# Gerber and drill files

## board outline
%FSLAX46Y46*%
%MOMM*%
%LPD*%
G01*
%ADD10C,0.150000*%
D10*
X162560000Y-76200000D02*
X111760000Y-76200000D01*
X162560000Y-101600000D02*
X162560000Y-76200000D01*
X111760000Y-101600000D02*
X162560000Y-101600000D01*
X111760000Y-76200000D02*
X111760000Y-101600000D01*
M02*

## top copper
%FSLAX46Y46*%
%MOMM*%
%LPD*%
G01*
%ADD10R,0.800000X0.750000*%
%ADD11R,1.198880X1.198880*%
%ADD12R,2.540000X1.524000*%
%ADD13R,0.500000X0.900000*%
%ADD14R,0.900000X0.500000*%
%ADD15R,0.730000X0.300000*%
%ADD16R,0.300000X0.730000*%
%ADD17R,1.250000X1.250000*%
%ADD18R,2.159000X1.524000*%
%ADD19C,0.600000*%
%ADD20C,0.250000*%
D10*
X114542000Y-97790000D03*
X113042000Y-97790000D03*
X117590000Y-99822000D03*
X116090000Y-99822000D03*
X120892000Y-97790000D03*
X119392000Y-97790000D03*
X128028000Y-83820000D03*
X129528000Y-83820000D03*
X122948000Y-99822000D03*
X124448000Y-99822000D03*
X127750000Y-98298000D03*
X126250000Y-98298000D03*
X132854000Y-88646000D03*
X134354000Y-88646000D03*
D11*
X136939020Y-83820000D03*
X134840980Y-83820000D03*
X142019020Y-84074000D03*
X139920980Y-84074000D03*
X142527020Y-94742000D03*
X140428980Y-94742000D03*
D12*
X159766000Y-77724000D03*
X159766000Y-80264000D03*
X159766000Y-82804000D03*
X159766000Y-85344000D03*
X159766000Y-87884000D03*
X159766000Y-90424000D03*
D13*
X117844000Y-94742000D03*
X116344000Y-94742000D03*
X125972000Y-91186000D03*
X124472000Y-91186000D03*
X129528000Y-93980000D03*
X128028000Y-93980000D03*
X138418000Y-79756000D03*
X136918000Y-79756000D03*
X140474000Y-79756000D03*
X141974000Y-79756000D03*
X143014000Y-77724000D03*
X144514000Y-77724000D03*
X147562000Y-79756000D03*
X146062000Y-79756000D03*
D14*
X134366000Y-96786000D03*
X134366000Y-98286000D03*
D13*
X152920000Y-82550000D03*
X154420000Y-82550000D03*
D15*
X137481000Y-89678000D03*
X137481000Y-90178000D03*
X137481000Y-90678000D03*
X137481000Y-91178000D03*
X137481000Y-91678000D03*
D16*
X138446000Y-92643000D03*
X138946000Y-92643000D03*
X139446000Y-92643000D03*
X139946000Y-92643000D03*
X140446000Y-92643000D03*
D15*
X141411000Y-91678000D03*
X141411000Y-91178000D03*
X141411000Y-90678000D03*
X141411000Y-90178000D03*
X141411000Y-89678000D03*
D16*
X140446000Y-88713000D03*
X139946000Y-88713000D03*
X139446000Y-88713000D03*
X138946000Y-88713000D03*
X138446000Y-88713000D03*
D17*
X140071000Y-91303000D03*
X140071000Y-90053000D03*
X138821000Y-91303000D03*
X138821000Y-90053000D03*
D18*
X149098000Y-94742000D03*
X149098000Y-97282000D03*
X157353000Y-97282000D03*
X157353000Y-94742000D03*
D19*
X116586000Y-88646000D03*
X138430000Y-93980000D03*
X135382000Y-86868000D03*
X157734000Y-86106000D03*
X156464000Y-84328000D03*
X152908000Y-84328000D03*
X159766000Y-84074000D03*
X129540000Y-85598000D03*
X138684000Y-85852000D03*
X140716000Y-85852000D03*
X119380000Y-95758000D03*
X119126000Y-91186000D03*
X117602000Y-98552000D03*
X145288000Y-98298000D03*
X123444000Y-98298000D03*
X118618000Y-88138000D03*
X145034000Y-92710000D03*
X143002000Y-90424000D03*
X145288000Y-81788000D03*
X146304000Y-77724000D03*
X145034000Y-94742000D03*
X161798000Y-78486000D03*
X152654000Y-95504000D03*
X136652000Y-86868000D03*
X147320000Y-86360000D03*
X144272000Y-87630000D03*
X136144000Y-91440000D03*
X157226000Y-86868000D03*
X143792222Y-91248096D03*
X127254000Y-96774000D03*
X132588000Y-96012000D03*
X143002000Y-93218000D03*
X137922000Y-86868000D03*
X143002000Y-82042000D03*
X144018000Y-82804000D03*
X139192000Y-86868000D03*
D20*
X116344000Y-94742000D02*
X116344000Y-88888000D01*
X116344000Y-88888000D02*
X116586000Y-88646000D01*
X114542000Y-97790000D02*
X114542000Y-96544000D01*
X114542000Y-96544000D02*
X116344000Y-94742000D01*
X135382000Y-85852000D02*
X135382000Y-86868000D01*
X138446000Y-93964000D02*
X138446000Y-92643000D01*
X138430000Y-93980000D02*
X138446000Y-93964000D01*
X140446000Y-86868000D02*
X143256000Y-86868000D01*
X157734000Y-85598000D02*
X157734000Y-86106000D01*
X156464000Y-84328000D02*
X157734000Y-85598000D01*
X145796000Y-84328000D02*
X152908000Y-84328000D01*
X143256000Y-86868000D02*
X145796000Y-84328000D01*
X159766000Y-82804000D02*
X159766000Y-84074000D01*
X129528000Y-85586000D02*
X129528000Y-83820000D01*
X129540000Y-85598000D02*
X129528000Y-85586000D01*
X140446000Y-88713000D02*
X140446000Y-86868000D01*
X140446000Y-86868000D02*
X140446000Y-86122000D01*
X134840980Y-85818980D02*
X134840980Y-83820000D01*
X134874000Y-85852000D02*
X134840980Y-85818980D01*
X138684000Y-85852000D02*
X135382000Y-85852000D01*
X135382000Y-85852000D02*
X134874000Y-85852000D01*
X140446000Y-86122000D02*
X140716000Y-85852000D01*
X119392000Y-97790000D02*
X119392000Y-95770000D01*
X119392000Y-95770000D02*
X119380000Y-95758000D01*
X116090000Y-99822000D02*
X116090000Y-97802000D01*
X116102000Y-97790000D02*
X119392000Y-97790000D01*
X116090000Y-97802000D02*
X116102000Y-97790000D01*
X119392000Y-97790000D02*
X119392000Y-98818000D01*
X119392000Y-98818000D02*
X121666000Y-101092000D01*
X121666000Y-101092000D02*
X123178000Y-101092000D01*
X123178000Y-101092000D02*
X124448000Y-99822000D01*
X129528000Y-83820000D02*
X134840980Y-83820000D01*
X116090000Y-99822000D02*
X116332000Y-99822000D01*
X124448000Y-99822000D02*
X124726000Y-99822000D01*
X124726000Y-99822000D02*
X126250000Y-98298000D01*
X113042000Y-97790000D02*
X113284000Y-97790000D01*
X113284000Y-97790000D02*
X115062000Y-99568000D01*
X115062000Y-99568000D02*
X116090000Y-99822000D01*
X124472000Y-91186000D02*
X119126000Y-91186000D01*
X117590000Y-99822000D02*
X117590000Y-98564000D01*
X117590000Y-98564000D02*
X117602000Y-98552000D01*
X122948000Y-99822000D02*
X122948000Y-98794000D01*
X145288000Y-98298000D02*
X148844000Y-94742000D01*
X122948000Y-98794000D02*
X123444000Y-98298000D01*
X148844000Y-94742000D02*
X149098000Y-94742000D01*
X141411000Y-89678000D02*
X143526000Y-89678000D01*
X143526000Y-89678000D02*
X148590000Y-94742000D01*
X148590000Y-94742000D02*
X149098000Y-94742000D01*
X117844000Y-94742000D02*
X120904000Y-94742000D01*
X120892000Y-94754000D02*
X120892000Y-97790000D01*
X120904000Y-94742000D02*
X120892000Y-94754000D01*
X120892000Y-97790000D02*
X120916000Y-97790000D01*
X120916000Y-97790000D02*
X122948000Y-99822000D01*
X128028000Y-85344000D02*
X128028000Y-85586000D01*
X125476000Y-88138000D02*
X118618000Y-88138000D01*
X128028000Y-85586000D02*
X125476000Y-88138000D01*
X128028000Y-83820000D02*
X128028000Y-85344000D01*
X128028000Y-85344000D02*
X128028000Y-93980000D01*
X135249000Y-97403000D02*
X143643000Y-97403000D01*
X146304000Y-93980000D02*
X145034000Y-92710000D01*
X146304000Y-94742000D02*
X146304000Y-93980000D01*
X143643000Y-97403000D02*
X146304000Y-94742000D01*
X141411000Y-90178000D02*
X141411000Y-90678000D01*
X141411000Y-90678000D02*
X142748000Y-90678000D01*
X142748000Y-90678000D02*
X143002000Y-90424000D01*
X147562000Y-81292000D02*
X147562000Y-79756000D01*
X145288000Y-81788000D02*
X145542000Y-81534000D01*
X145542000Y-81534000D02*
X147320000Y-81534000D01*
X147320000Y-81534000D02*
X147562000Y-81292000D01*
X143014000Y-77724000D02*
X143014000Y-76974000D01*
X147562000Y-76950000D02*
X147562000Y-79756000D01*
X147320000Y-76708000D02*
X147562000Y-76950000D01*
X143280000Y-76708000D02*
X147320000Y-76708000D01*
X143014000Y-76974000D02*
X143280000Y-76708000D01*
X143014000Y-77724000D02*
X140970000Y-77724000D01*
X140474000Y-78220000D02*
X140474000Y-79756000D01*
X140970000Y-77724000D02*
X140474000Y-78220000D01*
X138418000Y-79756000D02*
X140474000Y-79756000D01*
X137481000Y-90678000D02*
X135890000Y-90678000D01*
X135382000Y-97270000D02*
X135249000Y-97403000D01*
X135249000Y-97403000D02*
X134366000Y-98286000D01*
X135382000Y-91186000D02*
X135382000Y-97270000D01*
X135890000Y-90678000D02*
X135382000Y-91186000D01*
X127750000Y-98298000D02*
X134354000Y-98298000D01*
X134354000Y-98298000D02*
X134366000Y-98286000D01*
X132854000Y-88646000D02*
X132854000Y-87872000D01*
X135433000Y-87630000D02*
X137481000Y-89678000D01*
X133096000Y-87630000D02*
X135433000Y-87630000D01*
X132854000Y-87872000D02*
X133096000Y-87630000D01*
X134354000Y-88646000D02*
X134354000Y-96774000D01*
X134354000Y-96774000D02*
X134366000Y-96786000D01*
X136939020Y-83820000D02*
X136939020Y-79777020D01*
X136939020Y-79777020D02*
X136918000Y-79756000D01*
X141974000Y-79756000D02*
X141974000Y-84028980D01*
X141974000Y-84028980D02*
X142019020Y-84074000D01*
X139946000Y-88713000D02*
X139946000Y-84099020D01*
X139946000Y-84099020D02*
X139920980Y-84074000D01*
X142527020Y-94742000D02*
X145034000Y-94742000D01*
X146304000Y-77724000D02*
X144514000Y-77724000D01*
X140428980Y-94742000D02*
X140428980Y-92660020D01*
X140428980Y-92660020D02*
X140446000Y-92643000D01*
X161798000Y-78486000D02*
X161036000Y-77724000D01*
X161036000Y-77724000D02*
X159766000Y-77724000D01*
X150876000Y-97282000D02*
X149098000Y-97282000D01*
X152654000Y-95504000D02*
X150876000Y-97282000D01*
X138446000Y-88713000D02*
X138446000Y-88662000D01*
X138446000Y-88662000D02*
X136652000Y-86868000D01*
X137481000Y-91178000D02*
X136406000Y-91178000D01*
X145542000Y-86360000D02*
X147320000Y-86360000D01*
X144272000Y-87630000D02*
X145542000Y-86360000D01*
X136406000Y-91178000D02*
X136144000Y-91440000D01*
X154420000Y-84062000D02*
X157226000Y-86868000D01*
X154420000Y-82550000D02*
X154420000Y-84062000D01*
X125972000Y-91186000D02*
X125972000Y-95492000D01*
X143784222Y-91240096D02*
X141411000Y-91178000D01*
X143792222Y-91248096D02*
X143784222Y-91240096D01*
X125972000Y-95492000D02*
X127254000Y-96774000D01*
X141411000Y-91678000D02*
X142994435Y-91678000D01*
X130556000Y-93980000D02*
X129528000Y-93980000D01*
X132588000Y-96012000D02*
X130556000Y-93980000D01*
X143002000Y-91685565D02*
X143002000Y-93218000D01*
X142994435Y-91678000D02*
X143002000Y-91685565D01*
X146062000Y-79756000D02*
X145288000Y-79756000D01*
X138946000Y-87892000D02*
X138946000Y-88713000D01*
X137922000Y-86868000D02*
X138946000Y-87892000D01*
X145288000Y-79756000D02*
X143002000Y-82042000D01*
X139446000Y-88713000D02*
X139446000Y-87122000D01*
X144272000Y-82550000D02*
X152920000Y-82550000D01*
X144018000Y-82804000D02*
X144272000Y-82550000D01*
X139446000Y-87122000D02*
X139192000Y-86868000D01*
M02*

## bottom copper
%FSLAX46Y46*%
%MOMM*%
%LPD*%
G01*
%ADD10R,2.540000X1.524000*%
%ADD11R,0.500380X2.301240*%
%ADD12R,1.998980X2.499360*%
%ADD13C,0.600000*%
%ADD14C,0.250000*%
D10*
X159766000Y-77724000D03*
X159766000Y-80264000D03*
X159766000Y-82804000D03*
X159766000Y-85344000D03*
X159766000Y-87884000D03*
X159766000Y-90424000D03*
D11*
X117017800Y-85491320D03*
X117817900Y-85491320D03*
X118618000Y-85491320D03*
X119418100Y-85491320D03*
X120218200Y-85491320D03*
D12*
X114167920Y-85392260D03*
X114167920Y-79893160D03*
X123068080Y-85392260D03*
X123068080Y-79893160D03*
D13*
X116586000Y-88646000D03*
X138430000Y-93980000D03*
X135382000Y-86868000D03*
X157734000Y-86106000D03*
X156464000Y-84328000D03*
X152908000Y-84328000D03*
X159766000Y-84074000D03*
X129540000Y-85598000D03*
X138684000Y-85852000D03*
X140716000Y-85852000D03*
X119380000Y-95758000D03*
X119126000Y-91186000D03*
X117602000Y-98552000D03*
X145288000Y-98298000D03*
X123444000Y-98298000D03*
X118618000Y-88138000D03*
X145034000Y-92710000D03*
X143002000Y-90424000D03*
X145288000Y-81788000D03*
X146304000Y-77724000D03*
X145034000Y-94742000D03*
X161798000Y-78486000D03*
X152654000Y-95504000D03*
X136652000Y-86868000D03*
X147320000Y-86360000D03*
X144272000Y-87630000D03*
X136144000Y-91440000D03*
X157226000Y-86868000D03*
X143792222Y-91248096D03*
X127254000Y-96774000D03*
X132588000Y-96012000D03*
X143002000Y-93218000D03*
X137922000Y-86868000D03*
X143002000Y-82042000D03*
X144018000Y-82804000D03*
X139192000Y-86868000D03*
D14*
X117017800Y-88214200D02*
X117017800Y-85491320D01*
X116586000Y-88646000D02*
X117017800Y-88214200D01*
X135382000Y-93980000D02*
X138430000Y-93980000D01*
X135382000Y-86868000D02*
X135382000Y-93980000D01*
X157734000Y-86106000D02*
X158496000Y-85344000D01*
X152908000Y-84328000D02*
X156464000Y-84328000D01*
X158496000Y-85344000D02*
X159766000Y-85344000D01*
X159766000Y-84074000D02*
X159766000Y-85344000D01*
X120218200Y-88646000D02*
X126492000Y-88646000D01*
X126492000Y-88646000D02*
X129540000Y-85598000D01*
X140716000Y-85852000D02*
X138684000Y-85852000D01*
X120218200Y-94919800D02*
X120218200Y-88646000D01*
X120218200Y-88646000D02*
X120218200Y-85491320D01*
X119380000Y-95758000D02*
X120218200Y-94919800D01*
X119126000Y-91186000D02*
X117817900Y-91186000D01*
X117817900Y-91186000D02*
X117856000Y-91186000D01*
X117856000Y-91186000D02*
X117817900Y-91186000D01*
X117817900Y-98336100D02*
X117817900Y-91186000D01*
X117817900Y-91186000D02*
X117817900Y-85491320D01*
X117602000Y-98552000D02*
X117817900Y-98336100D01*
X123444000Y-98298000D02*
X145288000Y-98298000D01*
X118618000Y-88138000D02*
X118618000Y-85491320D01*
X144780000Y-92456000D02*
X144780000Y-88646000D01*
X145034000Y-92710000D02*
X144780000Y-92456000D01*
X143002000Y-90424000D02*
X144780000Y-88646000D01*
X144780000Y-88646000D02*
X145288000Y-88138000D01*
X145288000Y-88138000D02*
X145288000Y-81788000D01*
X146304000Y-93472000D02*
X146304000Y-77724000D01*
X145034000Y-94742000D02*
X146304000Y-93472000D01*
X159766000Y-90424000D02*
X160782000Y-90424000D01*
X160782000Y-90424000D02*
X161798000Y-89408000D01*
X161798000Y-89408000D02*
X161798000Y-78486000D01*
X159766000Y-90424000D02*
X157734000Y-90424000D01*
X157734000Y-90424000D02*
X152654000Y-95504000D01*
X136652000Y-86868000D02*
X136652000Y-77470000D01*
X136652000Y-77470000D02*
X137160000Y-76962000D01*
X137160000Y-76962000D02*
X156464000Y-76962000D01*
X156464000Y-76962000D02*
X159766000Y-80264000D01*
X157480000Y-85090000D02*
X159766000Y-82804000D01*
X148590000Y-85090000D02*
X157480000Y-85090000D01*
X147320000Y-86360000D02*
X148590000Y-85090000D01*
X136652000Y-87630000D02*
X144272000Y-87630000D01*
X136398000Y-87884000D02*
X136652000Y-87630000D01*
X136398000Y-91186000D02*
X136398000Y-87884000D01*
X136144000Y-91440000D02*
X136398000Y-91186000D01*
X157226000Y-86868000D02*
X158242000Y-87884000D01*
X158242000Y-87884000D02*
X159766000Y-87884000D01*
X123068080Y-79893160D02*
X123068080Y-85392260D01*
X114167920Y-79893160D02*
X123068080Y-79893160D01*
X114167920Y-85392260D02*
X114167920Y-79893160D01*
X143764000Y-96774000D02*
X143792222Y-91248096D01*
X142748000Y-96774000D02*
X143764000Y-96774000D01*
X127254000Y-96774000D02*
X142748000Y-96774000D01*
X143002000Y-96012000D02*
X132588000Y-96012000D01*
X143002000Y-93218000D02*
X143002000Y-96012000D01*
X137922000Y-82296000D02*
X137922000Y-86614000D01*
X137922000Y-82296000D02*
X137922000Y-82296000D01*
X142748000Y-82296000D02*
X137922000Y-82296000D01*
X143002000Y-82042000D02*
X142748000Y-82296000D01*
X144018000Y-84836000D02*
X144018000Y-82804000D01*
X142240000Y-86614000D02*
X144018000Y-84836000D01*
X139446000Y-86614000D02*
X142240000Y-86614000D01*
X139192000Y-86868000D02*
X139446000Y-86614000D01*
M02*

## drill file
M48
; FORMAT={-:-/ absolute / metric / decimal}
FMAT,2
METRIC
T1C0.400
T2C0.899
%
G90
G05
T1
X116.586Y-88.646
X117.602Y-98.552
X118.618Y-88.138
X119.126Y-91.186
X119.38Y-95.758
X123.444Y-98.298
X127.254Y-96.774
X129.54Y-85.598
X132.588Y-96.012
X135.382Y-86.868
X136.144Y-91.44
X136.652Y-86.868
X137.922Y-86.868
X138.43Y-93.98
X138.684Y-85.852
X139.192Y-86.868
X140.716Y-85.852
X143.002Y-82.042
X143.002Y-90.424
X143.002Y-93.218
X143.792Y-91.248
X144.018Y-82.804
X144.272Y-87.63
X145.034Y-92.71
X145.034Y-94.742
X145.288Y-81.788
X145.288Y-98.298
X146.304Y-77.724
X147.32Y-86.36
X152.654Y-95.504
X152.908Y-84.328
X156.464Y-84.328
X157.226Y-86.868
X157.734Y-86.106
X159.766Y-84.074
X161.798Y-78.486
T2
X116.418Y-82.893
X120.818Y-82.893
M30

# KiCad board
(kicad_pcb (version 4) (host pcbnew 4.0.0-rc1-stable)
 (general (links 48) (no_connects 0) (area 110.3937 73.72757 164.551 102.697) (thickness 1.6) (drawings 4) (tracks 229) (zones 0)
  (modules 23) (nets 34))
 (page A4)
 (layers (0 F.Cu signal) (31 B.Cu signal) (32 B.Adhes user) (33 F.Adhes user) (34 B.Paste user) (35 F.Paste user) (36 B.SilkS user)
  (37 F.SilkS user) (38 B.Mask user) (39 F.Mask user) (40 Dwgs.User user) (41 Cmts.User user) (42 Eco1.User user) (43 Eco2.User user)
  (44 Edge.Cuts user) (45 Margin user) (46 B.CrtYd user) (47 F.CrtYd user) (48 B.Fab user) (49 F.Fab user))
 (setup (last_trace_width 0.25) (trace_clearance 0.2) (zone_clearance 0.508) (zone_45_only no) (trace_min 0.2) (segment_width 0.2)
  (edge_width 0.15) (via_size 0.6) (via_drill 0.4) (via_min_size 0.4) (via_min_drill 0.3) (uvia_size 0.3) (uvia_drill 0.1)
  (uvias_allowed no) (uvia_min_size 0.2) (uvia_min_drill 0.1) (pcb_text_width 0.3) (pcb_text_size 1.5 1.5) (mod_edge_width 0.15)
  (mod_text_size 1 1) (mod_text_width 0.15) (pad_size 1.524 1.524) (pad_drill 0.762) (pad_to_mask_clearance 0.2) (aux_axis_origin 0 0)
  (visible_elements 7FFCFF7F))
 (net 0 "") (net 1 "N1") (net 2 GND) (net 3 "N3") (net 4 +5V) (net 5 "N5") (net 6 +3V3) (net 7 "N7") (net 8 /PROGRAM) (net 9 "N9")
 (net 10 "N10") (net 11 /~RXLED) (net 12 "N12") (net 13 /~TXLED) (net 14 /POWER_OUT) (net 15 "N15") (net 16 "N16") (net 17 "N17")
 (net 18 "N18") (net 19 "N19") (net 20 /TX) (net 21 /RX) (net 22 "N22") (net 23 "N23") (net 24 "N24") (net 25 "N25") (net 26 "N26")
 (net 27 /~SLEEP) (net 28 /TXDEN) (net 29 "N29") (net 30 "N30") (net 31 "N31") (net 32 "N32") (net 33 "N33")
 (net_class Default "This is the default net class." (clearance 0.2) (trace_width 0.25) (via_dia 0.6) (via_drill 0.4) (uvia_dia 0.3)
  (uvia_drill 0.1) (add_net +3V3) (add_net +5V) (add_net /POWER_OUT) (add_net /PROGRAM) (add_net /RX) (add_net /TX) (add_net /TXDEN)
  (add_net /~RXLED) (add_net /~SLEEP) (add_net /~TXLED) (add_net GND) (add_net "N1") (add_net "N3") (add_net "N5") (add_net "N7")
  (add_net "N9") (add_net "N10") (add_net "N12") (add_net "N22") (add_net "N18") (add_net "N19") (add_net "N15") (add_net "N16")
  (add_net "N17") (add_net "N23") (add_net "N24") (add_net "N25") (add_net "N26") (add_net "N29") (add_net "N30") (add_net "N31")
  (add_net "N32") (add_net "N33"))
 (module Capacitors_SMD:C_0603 (layer F.Cu) (at 113.792 97.79 180)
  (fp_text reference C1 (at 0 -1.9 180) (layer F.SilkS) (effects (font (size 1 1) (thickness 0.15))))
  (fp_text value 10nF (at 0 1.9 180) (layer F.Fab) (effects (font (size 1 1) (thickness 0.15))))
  (pad 1 smd rect (at -0.75 0 180) (size 0.8 0.75) (layers F.Cu F.Paste F.Mask) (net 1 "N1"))
  (pad 2 smd rect (at 0.75 0 180) (size 0.8 0.75) (layers F.Cu F.Paste F.Mask) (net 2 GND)))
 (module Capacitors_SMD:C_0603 (layer F.Cu) (at 116.84 99.822 180)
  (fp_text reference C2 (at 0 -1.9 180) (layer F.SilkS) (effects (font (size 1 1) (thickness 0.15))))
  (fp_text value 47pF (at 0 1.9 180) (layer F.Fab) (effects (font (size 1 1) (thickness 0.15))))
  (pad 1 smd rect (at -0.75 0 180) (size 0.8 0.75) (layers F.Cu F.Paste F.Mask) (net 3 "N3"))
  (pad 2 smd rect (at 0.75 0 180) (size 0.8 0.75) (layers F.Cu F.Paste F.Mask) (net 2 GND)))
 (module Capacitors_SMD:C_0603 (layer F.Cu) (at 120.142 97.79 180)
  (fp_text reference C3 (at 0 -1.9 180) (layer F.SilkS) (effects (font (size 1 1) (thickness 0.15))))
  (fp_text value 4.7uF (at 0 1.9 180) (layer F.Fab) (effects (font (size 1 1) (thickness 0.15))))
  (pad 1 smd rect (at -0.75 0 180) (size 0.8 0.75) (layers F.Cu F.Paste F.Mask) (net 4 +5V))
  (pad 2 smd rect (at 0.75 0 180) (size 0.8 0.75) (layers F.Cu F.Paste F.Mask) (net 2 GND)))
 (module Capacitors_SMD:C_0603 (layer F.Cu) (at 128.778 83.82)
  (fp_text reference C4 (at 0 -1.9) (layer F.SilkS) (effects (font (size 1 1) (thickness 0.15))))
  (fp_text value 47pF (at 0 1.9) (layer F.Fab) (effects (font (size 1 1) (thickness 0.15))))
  (pad 1 smd rect (at -0.75 0) (size 0.8 0.75) (layers F.Cu F.Paste F.Mask) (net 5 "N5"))
  (pad 2 smd rect (at 0.75 0) (size 0.8 0.75) (layers F.Cu F.Paste F.Mask) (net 2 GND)))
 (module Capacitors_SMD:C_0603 (layer F.Cu) (at 123.698 99.822)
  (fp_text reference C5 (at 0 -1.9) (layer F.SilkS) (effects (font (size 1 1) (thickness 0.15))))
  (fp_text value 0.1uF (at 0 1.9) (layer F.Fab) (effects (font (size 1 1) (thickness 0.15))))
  (pad 1 smd rect (at -0.75 0) (size 0.8 0.75) (layers F.Cu F.Paste F.Mask) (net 4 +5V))
  (pad 2 smd rect (at 0.75 0) (size 0.8 0.75) (layers F.Cu F.Paste F.Mask) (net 2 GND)))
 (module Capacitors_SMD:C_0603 (layer F.Cu) (at 127 98.298 180)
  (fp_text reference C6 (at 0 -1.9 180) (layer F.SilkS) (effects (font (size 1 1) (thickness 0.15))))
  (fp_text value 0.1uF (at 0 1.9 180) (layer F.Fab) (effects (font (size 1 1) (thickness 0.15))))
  (pad 1 smd rect (at -0.75 0 180) (size 0.8 0.75) (layers F.Cu F.Paste F.Mask) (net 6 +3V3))
  (pad 2 smd rect (at 0.75 0 180) (size 0.8 0.75) (layers F.Cu F.Paste F.Mask) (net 2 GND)))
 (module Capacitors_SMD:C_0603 (layer F.Cu) (at 133.604 88.646)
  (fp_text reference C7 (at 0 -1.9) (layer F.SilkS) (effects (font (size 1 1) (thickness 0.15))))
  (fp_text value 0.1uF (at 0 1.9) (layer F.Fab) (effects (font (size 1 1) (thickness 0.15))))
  (pad 1 smd rect (at -0.75 0) (size 0.8 0.75) (layers F.Cu F.Paste F.Mask) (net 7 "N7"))
  (pad 2 smd rect (at 0.75 0) (size 0.8 0.75) (layers F.Cu F.Paste F.Mask) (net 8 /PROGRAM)))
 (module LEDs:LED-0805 (layer F.Cu) (at 135.89 83.82)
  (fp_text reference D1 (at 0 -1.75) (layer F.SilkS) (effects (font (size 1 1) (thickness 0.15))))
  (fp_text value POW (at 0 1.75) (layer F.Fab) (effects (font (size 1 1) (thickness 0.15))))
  (pad 2 smd rect (at 1.04902 0 180) (size 1.19888 1.19888) (layers F.Cu F.Paste F.Mask) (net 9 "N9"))
  (pad 1 smd rect (at -1.04902 0 180) (size 1.19888 1.19888) (layers F.Cu F.Paste F.Mask) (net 2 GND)))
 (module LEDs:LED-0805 (layer F.Cu) (at 140.97 84.074)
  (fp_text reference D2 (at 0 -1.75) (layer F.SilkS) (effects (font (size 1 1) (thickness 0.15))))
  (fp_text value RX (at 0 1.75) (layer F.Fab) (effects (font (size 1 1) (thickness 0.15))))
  (pad 2 smd rect (at 1.04902 0 180) (size 1.19888 1.19888) (layers F.Cu F.Paste F.Mask) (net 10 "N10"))
  (pad 1 smd rect (at -1.04902 0 180) (size 1.19888 1.19888) (layers F.Cu F.Paste F.Mask) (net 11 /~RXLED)))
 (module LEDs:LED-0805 (layer F.Cu) (at 141.478 94.742)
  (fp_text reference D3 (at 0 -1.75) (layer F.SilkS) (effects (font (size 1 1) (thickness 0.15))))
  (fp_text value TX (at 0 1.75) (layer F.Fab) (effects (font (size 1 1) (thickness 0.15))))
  (pad 2 smd rect (at 1.04902 0 180) (size 1.19888 1.19888) (layers F.Cu F.Paste F.Mask) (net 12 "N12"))
  (pad 1 smd rect (at -1.04902 0 180) (size 1.19888 1.19888) (layers F.Cu F.Paste F.Mask) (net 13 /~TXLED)))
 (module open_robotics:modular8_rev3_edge (layer F.Cu) (at 159.766 82.804 270)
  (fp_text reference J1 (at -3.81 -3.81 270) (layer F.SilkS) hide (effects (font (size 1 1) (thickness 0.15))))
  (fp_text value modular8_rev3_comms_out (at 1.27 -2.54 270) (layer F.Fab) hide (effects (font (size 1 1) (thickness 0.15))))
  (pad 1 smd rect (at -5.08 0 270) (size 1.524 2.54) (layers F.Cu F.Paste F.Mask) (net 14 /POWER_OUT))
  (pad 3 smd rect (at -2.54 0 270) (size 1.524 2.54) (layers F.Cu F.Paste F.Mask) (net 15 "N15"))
  (pad 5 smd rect (at 0 0 270) (size 1.524 2.54) (layers F.Cu F.Paste F.Mask) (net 2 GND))
  (pad 7 smd rect (at 2.54 0 270) (size 1.524 2.54) (layers F.Cu F.Paste F.Mask) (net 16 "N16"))
  (pad 9 smd rect (at 5.08 0 270) (size 1.524 2.54) (layers F.Cu F.Paste F.Mask) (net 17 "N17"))
  (pad 11 smd rect (at 7.62 0 270) (size 1.524 2.54) (layers F.Cu F.Paste F.Mask) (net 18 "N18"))
  (pad 2 smd rect (at -5.08 0 270) (size 1.524 2.54) (layers B.Cu F.Paste F.Mask) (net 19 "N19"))
  (pad 4 smd rect (at -2.54 0 270) (size 1.524 2.54) (layers B.Cu F.Paste F.Mask) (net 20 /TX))
  (pad 6 smd rect (at 0 0 270) (size 1.524 2.54) (layers B.Cu F.Paste F.Mask) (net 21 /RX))
  (pad 8 smd rect (at 2.54 0 270) (size 1.524 2.54) (layers B.Cu F.Paste F.Mask) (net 2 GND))
  (pad 10 smd rect (at 5.08 0 270) (size 1.524 2.54) (layers B.Cu F.Paste F.Mask) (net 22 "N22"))
  (pad 12 smd rect (at 7.62 0 270) (size 1.524 2.54) (layers B.Cu F.Paste F.Mask) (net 14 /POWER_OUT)))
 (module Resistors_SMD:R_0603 (layer F.Cu) (at 117.094 94.742 180)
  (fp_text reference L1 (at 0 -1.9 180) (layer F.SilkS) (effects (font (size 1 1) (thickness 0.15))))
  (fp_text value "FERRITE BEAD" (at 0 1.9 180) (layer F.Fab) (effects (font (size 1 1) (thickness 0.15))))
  (pad 1 smd rect (at -0.75 0 180) (size 0.5 0.9) (layers F.Cu F.Paste F.Mask) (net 4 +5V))
  (pad 2 smd rect (at 0.75 0 180) (size 0.5 0.9) (layers F.Cu F.Paste F.Mask) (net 1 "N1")))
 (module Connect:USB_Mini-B (layer B.Cu) (at 118.618 82.042 270)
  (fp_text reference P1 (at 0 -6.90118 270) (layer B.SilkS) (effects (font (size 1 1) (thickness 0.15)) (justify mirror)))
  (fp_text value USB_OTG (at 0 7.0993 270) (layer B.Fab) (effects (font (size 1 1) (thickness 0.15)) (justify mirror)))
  (pad 1 smd rect (at 3.44932 1.6002 270) (size 2.30124 0.50038) (layers B.Cu B.Paste B.Mask) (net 1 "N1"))
  (pad 2 smd rect (at 3.44932 0.8001 270) (size 2.30124 0.50038) (layers B.Cu B.Paste B.Mask) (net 3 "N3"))
  (pad 3 smd rect (at 3.44932 0 270) (size 2.30124 0.50038) (layers B.Cu B.Paste B.Mask) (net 5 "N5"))
  (pad 4 smd rect (at 3.44932 -0.8001 270) (size 2.30124 0.50038) (layers B.Cu B.Paste B.Mask) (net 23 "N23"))
  (pad 5 smd rect (at 3.44932 -1.6002 270) (size 2.30124 0.50038) (layers B.Cu B.Paste B.Mask) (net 2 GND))
  (pad 6 smd rect (at 3.35026 4.45008 270) (size 2.49936 1.99898) (layers B.Cu B.Paste B.Mask) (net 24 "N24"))
  (pad 6 smd rect (at -2.14884 4.45008 270) (size 2.49936 1.99898) (layers B.Cu B.Paste B.Mask) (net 24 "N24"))
  (pad 6 smd rect (at 3.35026 -4.45008 270) (size 2.49936 1.99898) (layers B.Cu B.Paste B.Mask) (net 24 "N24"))
  (pad 6 smd rect (at -2.14884 -4.45008 270) (size 2.49936 1.99898) (layers B.Cu B.Paste B.Mask) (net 24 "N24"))
  (pad "" np_thru_hole circle (at 0.8509 2.19964 270) (size 0.89916 0.89916) (drill 0.89916) (layers *.Cu *.Mask B.SilkS))
  (pad "" np_thru_hole circle (at 0.8509 -2.19964 270) (size 0.89916 0.89916) (drill 0.89916) (layers *.Cu *.Mask B.SilkS)))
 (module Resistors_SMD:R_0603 (layer F.Cu) (at 125.222 91.186 180)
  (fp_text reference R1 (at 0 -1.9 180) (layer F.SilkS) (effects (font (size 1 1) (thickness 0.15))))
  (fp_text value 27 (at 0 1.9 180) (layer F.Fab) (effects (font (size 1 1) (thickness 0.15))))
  (pad 1 smd rect (at -0.75 0 180) (size 0.5 0.9) (layers F.Cu F.Paste F.Mask) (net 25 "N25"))
  (pad 2 smd rect (at 0.75 0 180) (size 0.5 0.9) (layers F.Cu F.Paste F.Mask) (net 3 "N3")))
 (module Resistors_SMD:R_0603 (layer F.Cu) (at 128.778 93.98 180)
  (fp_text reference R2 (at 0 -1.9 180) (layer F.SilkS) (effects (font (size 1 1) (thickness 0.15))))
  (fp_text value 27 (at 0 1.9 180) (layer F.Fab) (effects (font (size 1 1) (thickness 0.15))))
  (pad 1 smd rect (at -0.75 0 180) (size 0.5 0.9) (layers F.Cu F.Paste F.Mask) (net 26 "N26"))
  (pad 2 smd rect (at 0.75 0 180) (size 0.5 0.9) (layers F.Cu F.Paste F.Mask) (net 5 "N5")))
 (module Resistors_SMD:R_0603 (layer F.Cu) (at 137.668 79.756 180)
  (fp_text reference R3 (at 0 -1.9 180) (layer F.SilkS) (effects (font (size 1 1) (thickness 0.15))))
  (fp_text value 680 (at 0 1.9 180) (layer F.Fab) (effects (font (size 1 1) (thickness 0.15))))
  (pad 1 smd rect (at -0.75 0 180) (size 0.5 0.9) (layers F.Cu F.Paste F.Mask) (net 6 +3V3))
  (pad 2 smd rect (at 0.75 0 180) (size 0.5 0.9) (layers F.Cu F.Paste F.Mask) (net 9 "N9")))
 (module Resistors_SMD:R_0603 (layer F.Cu) (at 141.224 79.756)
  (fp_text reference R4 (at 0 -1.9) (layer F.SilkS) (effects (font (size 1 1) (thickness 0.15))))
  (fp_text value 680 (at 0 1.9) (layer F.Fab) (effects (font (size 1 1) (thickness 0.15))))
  (pad 1 smd rect (at -0.75 0) (size 0.5 0.9) (layers F.Cu F.Paste F.Mask) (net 6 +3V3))
  (pad 2 smd rect (at 0.75 0) (size 0.5 0.9) (layers F.Cu F.Paste F.Mask) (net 10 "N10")))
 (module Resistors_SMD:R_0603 (layer F.Cu) (at 143.764 77.724)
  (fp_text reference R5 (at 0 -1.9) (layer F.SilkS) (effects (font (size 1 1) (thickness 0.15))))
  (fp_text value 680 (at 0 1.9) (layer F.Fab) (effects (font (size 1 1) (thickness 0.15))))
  (pad 1 smd rect (at -0.75 0) (size 0.5 0.9) (layers F.Cu F.Paste F.Mask) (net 6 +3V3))
  (pad 2 smd rect (at 0.75 0) (size 0.5 0.9) (layers F.Cu F.Paste F.Mask) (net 12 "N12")))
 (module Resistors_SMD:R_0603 (layer F.Cu) (at 146.812 79.756 180)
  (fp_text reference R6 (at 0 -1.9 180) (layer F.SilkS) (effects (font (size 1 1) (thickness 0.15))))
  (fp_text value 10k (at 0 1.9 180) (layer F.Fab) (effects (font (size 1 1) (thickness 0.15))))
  (pad 1 smd rect (at -0.75 0 180) (size 0.5 0.9) (layers F.Cu F.Paste F.Mask) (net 6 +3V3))
  (pad 2 smd rect (at 0.75 0 180) (size 0.5 0.9) (layers F.Cu F.Paste F.Mask) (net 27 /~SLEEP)))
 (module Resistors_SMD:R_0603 (layer F.Cu) (at 134.366 97.536 270)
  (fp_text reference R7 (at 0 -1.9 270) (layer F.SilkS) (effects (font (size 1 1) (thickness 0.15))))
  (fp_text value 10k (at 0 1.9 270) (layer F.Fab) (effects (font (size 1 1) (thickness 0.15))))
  (pad 1 smd rect (at -0.75 0 270) (size 0.5 0.9) (layers F.Cu F.Paste F.Mask) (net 8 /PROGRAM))
  (pad 2 smd rect (at 0.75 0 270) (size 0.5 0.9) (layers F.Cu F.Paste F.Mask) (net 6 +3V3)))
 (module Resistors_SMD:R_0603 (layer F.Cu) (at 153.67 82.55)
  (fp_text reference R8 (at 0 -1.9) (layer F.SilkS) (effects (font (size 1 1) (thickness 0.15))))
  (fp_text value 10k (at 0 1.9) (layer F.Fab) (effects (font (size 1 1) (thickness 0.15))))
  (pad 1 smd rect (at -0.75 0) (size 0.5 0.9) (layers F.Cu F.Paste F.Mask) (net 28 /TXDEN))
  (pad 2 smd rect (at 0.75 0) (size 0.5 0.9) (layers F.Cu F.Paste F.Mask) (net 22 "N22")))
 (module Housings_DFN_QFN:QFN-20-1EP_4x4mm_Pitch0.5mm (layer F.Cu) (at 139.446 90.678)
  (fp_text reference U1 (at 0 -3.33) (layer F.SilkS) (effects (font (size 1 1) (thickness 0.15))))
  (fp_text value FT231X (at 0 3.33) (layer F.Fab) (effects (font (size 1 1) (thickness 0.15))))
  (pad 1 smd rect (at -1.965 -1) (size 0.73 0.3) (layers F.Cu F.Paste F.Mask) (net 7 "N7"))
  (pad 2 smd rect (at -1.965 -0.5) (size 0.73 0.3) (layers F.Cu F.Paste F.Mask) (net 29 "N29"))
  (pad 3 smd rect (at -1.965 0) (size 0.73 0.3) (layers F.Cu F.Paste F.Mask) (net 6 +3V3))
  (pad 4 smd rect (at -1.965 0.5) (size 0.73 0.3) (layers F.Cu F.Paste F.Mask) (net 21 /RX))
  (pad 5 smd rect (at -1.965 1) (size 0.73 0.3) (layers F.Cu F.Paste F.Mask) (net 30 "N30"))
  (pad 6 smd rect (at -1 1.965 90) (size 0.73 0.3) (layers F.Cu F.Paste F.Mask) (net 2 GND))
  (pad 7 smd rect (at -0.5 1.965 90) (size 0.73 0.3) (layers F.Cu F.Paste F.Mask) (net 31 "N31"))
  (pad 8 smd rect (at 0 1.965 90) (size 0.73 0.3) (layers F.Cu F.Paste F.Mask) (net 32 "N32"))
  (pad 9 smd rect (at 0.5 1.965 90) (size 0.73 0.3) (layers F.Cu F.Paste F.Mask) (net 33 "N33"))
  (pad 10 smd rect (at 1 1.965 90) (size 0.73 0.3) (layers F.Cu F.Paste F.Mask) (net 13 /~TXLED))
  (pad 11 smd rect (at 1.965 1) (size 0.73 0.3) (layers F.Cu F.Paste F.Mask) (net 26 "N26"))
  (pad 12 smd rect (at 1.965 0.5) (size 0.73 0.3) (layers F.Cu F.Paste F.Mask) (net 25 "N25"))
  (pad 13 smd rect (at 1.965 0) (size 0.73 0.3) (layers F.Cu F.Paste F.Mask) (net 6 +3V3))
  (pad 14 smd rect (at 1.965 -0.5) (size 0.73 0.3) (layers F.Cu F.Paste F.Mask) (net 6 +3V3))
  (pad 15 smd rect (at 1.965 -1) (size 0.73 0.3) (layers F.Cu F.Paste F.Mask) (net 4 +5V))
  (pad 16 smd rect (at 1 -1.965 90) (size 0.73 0.3) (layers F.Cu F.Paste F.Mask) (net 2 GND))
  (pad 17 smd rect (at 0.5 -1.965 90) (size 0.73 0.3) (layers F.Cu F.Paste F.Mask) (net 11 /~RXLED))
  (pad 18 smd rect (at 0 -1.965 90) (size 0.73 0.3) (layers F.Cu F.Paste F.Mask) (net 28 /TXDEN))
  (pad 19 smd rect (at -0.5 -1.965 90) (size 0.73 0.3) (layers F.Cu F.Paste F.Mask) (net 27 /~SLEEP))
  (pad 20 smd rect (at -1 -1.965 90) (size 0.73 0.3) (layers F.Cu F.Paste F.Mask) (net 20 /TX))
  (pad 21 smd rect (at 0.625 0.625) (size 1.25 1.25) (layers F.Cu F.Paste F.Mask) (solder_paste_margin_ratio -0.2))
  (pad 21 smd rect (at 0.625 -0.625) (size 1.25 1.25) (layers F.Cu F.Paste F.Mask) (solder_paste_margin_ratio -0.2))
  (pad 21 smd rect (at -0.625 0.625) (size 1.25 1.25) (layers F.Cu F.Paste F.Mask) (solder_paste_margin_ratio -0.2))
  (pad 21 smd rect (at -0.625 -0.625) (size 1.25 1.25) (layers F.Cu F.Paste F.Mask) (solder_paste_margin_ratio -0.2)))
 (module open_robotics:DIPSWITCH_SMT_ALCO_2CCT (layer F.Cu) (at 149.098 94.742)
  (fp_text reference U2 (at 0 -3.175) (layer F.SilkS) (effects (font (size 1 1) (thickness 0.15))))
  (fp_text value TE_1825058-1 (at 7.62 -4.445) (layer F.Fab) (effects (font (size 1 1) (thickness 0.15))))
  (pad 1 smd rect (at 0 0) (size 2.159 1.524) (layers F.Cu F.Paste F.Mask) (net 4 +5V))
  (pad 2 smd rect (at 0 2.54) (size 2.159 1.524) (layers F.Cu F.Paste F.Mask) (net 14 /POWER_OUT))
  (pad 3 smd rect (at 8.255 2.54) (size 2.159 1.524) (layers F.Cu F.Paste F.Mask))
  (pad 4 smd rect (at 8.255 0) (size 2.159 1.524) (layers F.Cu F.Paste F.Mask)))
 (gr_line (start 162.56 76.2) (end 111.76 76.2) (angle 90) (layer Edge.Cuts) (width 0.15))
 (gr_line (start 162.56 101.6) (end 162.56 76.2) (angle 90) (layer Edge.Cuts) (width 0.15))
 (gr_line (start 111.76 101.6) (end 162.56 101.6) (angle 90) (layer Edge.Cuts) (width 0.15))
 (gr_line (start 111.76 76.2) (end 111.76 101.6) (angle 90) (layer Edge.Cuts) (width 0.15))
 (segment (start 116.344 94.742) (end 116.344 88.888) (width 0.25) (layer F.Cu) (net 1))
 (segment (start 117.0178 88.2142) (end 117.0178 85.49132) (width 0.25) (layer B.Cu) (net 1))
 (segment (start 116.586 88.646) (end 117.0178 88.2142) (width 0.25) (layer B.Cu) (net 1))
 (via (at 116.586 88.646) (size 0.6) (drill 0.4) (layers F.Cu B.Cu) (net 1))
 (segment (start 116.344 88.888) (end 116.586 88.646) (width 0.25) (layer F.Cu) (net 1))
 (segment (start 114.542 97.79) (end 114.542 96.544) (width 0.25) (layer F.Cu) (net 1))
 (segment (start 114.542 96.544) (end 116.344 94.742) (width 0.25) (layer F.Cu) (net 1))
 (segment (start 135.382 85.852) (end 135.382 86.868) (width 0.25) (layer F.Cu) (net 2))
 (segment (start 138.446 93.964) (end 138.446 92.643) (width 0.25) (layer F.Cu) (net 2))
 (segment (start 138.43 93.98) (end 138.446 93.964) (width 0.25) (layer F.Cu) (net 2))
 (via (at 138.43 93.98) (size 0.6) (drill 0.4) (layers F.Cu B.Cu) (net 2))
 (segment (start 135.382 93.98) (end 138.43 93.98) (width 0.25) (layer B.Cu) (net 2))
 (segment (start 135.382 86.868) (end 135.382 93.98) (width 0.25) (layer B.Cu) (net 2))
 (via (at 135.382 86.868) (size 0.6) (drill 0.4) (layers F.Cu B.Cu) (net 2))
 (segment (start 140.446 86.868) (end 143.256 86.868) (width 0.25) (layer F.Cu) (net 2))
 (segment (start 157.734 86.106) (end 158.496 85.344) (width 0.25) (layer B.Cu) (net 2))
 (via (at 157.734 86.106) (size 0.6) (drill 0.4) (layers F.Cu B.Cu) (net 2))
 (segment (start 157.734 85.598) (end 157.734 86.106) (width 0.25) (layer F.Cu) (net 2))
 (segment (start 156.464 84.328) (end 157.734 85.598) (width 0.25) (layer F.Cu) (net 2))
 (via (at 156.464 84.328) (size 0.6) (drill 0.4) (layers F.Cu B.Cu) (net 2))
 (segment (start 152.908 84.328) (end 156.464 84.328) (width 0.25) (layer B.Cu) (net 2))
 (via (at 152.908 84.328) (size 0.6) (drill 0.4) (layers F.Cu B.Cu) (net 2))
 (segment (start 145.796 84.328) (end 152.908 84.328) (width 0.25) (layer F.Cu) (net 2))
 (segment (start 143.256 86.868) (end 145.796 84.328) (width 0.25) (layer F.Cu) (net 2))
 (segment (start 158.496 85.344) (end 159.766 85.344) (width 0.25) (layer B.Cu) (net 2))
 (segment (start 159.766 82.804) (end 159.766 84.074) (width 0.25) (layer F.Cu) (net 2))
 (segment (start 159.766 84.074) (end 159.766 85.344) (width 0.25) (layer B.Cu) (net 2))
 (via (at 159.766 84.074) (size 0.6) (drill 0.4) (layers F.Cu B.Cu) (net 2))
 (segment (start 120.2182 88.646) (end 126.492 88.646) (width 0.25) (layer B.Cu) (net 2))
 (segment (start 129.528 85.586) (end 129.528 83.82) (width 0.25) (layer F.Cu) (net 2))
 (segment (start 129.54 85.598) (end 129.528 85.586) (width 0.25) (layer F.Cu) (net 2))
 (via (at 129.54 85.598) (size 0.6) (drill 0.4) (layers F.Cu B.Cu) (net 2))
 (segment (start 126.492 88.646) (end 129.54 85.598) (width 0.25) (layer B.Cu) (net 2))
 (segment (start 140.446 88.713) (end 140.446 86.868) (width 0.25) (layer F.Cu) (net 2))
 (segment (start 140.446 86.868) (end 140.446 86.122) (width 0.25) (layer F.Cu) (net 2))
 (segment (start 134.84098 85.81898) (end 134.84098 83.82) (width 0.25) (layer F.Cu) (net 2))
 (segment (start 134.874 85.852) (end 134.84098 85.81898) (width 0.25) (layer F.Cu) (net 2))
 (segment (start 138.684 85.852) (end 135.382 85.852) (width 0.25) (layer F.Cu) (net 2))
 (segment (start 135.382 85.852) (end 134.874 85.852) (width 0.25) (layer F.Cu) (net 2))
 (via (at 138.684 85.852) (size 0.6) (drill 0.4) (layers F.Cu B.Cu) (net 2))
 (segment (start 140.716 85.852) (end 138.684 85.852) (width 0.25) (layer B.Cu) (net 2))
 (via (at 140.716 85.852) (size 0.6) (drill 0.4) (layers F.Cu B.Cu) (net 2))
 (segment (start 140.446 86.122) (end 140.716 85.852) (width 0.25) (layer F.Cu) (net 2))
 (segment (start 119.392 97.79) (end 119.392 95.77) (width 0.25) (layer F.Cu) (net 2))
 (segment (start 120.2182 94.9198) (end 120.2182 88.646) (width 0.25) (layer B.Cu) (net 2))
 (segment (start 120.2182 88.646) (end 120.2182 85.49132) (width 0.25) (layer B.Cu) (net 2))
 (segment (start 119.38 95.758) (end 120.2182 94.9198) (width 0.25) (layer B.Cu) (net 2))
 (via (at 119.38 95.758) (size 0.6) (drill 0.4) (layers F.Cu B.Cu) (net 2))
 (segment (start 119.392 95.77) (end 119.38 95.758) (width 0.25) (layer F.Cu) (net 2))
 (segment (start 116.09 99.822) (end 116.09 97.802) (width 0.25) (layer F.Cu) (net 2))
 (segment (start 116.102 97.79) (end 119.392 97.79) (width 0.25) (layer F.Cu) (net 2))
 (segment (start 116.09 97.802) (end 116.102 97.79) (width 0.25) (layer F.Cu) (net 2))
 (segment (start 119.392 97.79) (end 119.392 98.818) (width 0.25) (layer F.Cu) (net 2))
 (segment (start 119.392 98.818) (end 121.666 101.092) (width 0.25) (layer F.Cu) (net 2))
 (segment (start 121.666 101.092) (end 123.178 101.092) (width 0.25) (layer F.Cu) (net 2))
 (segment (start 123.178 101.092) (end 124.448 99.822) (width 0.25) (layer F.Cu) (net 2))
 (segment (start 129.528 83.82) (end 134.84098 83.82) (width 0.25) (layer F.Cu) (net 2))
 (segment (start 116.09 99.822) (end 116.332 99.822) (width 0.25) (layer F.Cu) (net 2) (status 30))
 (segment (start 124.448 99.822) (end 124.726 99.822) (width 0.25) (layer F.Cu) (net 2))
 (segment (start 124.726 99.822) (end 126.25 98.298) (width 0.25) (layer F.Cu) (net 2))
 (segment (start 113.042 97.79) (end 113.284 97.79) (width 0.25) (layer F.Cu) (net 2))
 (segment (start 113.284 97.79) (end 115.062 99.568) (width 0.25) (layer F.Cu) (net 2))
 (segment (start 115.062 99.568) (end 116.09 99.822) (width 0.25) (layer F.Cu) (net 2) (status 20))
 (segment (start 124.472 91.186) (end 119.126 91.186) (width 0.25) (layer F.Cu) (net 3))
 (segment (start 119.126 91.186) (end 117.8179 91.186) (width 0.25) (layer B.Cu) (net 3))
 (via (at 119.126 91.186) (size 0.6) (drill 0.4) (layers F.Cu B.Cu) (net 3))
 (segment (start 117.8179 91.186) (end 117.856 91.186) (width 0.25) (layer B.Cu) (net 3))
 (segment (start 117.856 91.186) (end 117.8179 91.186) (width 0.25) (layer B.Cu) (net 3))
 (segment (start 117.59 99.822) (end 117.59 98.564) (width 0.25) (layer F.Cu) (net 3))
 (segment (start 117.8179 98.3361) (end 117.8179 91.186) (width 0.25) (layer B.Cu) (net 3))
 (segment (start 117.8179 91.186) (end 117.8179 85.49132) (width 0.25) (layer B.Cu) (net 3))
 (segment (start 117.602 98.552) (end 117.8179 98.3361) (width 0.25) (layer B.Cu) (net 3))
 (via (at 117.602 98.552) (size 0.6) (drill 0.4) (layers F.Cu B.Cu) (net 3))
 (segment (start 117.59 98.564) (end 117.602 98.552) (width 0.25) (layer F.Cu) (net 3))
 (segment (start 122.948 99.822) (end 122.948 98.794) (width 0.25) (layer F.Cu) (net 4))
 (segment (start 145.288 98.298) (end 148.844 94.742) (width 0.25) (layer F.Cu) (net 4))
 (via (at 145.288 98.298) (size 0.6) (drill 0.4) (layers F.Cu B.Cu) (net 4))
 (segment (start 123.444 98.298) (end 145.288 98.298) (width 0.25) (layer B.Cu) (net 4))
 (via (at 123.444 98.298) (size 0.6) (drill 0.4) (layers F.Cu B.Cu) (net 4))
 (segment (start 122.948 98.794) (end 123.444 98.298) (width 0.25) (layer F.Cu) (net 4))
 (segment (start 148.844 94.742) (end 149.098 94.742) (width 0.25) (layer F.Cu) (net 4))
 (segment (start 141.411 89.678) (end 143.526 89.678) (width 0.25) (layer F.Cu) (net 4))
 (segment (start 143.526 89.678) (end 148.59 94.742) (width 0.25) (layer F.Cu) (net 4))
 (segment (start 148.59 94.742) (end 149.098 94.742) (width 0.25) (layer F.Cu) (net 4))
 (segment (start 117.844 94.742) (end 120.904 94.742) (width 0.25) (layer F.Cu) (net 4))
 (segment (start 120.892 94.754) (end 120.892 97.79) (width 0.25) (layer F.Cu) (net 4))
 (segment (start 120.904 94.742) (end 120.892 94.754) (width 0.25) (layer F.Cu) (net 4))
 (segment (start 120.892 97.79) (end 120.916 97.79) (width 0.25) (layer F.Cu) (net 4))
 (segment (start 120.916 97.79) (end 122.948 99.822) (width 0.25) (layer F.Cu) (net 4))
 (segment (start 128.028 85.344) (end 128.028 85.586) (width 0.25) (layer F.Cu) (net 5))
 (segment (start 118.618 88.138) (end 118.618 85.49132) (width 0.25) (layer B.Cu) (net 5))
 (via (at 118.618 88.138) (size 0.6) (drill 0.4) (layers F.Cu B.Cu) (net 5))
 (segment (start 125.476 88.138) (end 118.618 88.138) (width 0.25) (layer F.Cu) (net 5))
 (segment (start 128.028 85.586) (end 125.476 88.138) (width 0.25) (layer F.Cu) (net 5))
 (segment (start 128.028 83.82) (end 128.028 85.344) (width 0.25) (layer F.Cu) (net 5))
 (segment (start 128.028 85.344) (end 128.028 93.98) (width 0.25) (layer F.Cu) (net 5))
 (segment (start 135.249 97.403) (end 143.643 97.403) (width 0.25) (layer F.Cu) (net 6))
 (segment (start 144.78 92.456) (end 144.78 88.646) (width 0.25) (layer B.Cu) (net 6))
 (segment (start 145.034 92.71) (end 144.78 92.456) (width 0.25) (layer B.Cu) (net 6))
 (via (at 145.034 92.71) (size 0.6) (drill 0.4) (layers F.Cu B.Cu) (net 6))
 (segment (start 146.304 93.98) (end 145.034 92.71) (width 0.25) (layer F.Cu) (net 6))
 (segment (start 146.304 94.742) (end 146.304 93.98) (width 0.25) (layer F.Cu) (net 6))
 (segment (start 143.643 97.403) (end 146.304 94.742) (width 0.25) (layer F.Cu) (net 6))
 (segment (start 141.411 90.178) (end 141.411 90.678) (width 0.25) (layer F.Cu) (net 6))
 (segment (start 141.411 90.678) (end 142.748 90.678) (width 0.25) (layer F.Cu) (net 6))
 (segment (start 142.748 90.678) (end 143.002 90.424) (width 0.25) (layer F.Cu) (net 6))
 (via (at 143.002 90.424) (size 0.6) (drill 0.4) (layers F.Cu B.Cu) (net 6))
 (segment (start 143.002 90.424) (end 144.78 88.646) (width 0.25) (layer B.Cu) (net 6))
 (segment (start 147.562 81.292) (end 147.562 79.756) (width 0.25) (layer F.Cu) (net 6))
 (segment (start 144.78 88.646) (end 145.288 88.138) (width 0.25) (layer B.Cu) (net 6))
 (segment (start 145.288 88.138) (end 145.288 81.788) (width 0.25) (layer B.Cu) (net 6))
 (via (at 145.288 81.788) (size 0.6) (drill 0.4) (layers F.Cu B.Cu) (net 6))
 (segment (start 145.288 81.788) (end 145.542 81.534) (width 0.25) (layer F.Cu) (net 6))
 (segment (start 145.542 81.534) (end 147.32 81.534) (width 0.25) (layer F.Cu) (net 6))
 (segment (start 147.32 81.534) (end 147.562 81.292) (width 0.25) (layer F.Cu) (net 6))
 (segment (start 143.014 77.724) (end 143.014 76.974) (width 0.25) (layer F.Cu) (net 6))
 (segment (start 147.562 76.95) (end 147.562 79.756) (width 0.25) (layer F.Cu) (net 6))
 (segment (start 147.32 76.708) (end 147.562 76.95) (width 0.25) (layer F.Cu) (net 6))
 (segment (start 143.28 76.708) (end 147.32 76.708) (width 0.25) (layer F.Cu) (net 6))
 (segment (start 143.014 76.974) (end 143.28 76.708) (width 0.25) (layer F.Cu) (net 6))
 (segment (start 143.014 77.724) (end 140.97 77.724) (width 0.25) (layer F.Cu) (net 6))
 (segment (start 140.474 78.22) (end 140.474 79.756) (width 0.25) (layer F.Cu) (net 6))
 (segment (start 140.97 77.724) (end 140.474 78.22) (width 0.25) (layer F.Cu) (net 6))
 (segment (start 138.418 79.756) (end 140.474 79.756) (width 0.25) (layer F.Cu) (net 6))
 (segment (start 137.481 90.678) (end 135.89 90.678) (width 0.25) (layer F.Cu) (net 6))
 (segment (start 135.382 97.27) (end 135.249 97.403) (width 0.25) (layer F.Cu) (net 6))
 (segment (start 135.249 97.403) (end 134.366 98.286) (width 0.25) (layer F.Cu) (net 6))
 (segment (start 135.382 91.186) (end 135.382 97.27) (width 0.25) (layer F.Cu) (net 6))
 (segment (start 135.89 90.678) (end 135.382 91.186) (width 0.25) (layer F.Cu) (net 6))
 (segment (start 127.75 98.298) (end 134.354 98.298) (width 0.25) (layer F.Cu) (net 6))
 (segment (start 134.354 98.298) (end 134.366 98.286) (width 0.25) (layer F.Cu) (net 6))
 (segment (start 132.854 88.646) (end 132.854 87.872) (width 0.25) (layer F.Cu) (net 7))
 (segment (start 135.433 87.63) (end 137.481 89.678) (width 0.25) (layer F.Cu) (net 7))
 (segment (start 133.096 87.63) (end 135.433 87.63) (width 0.25) (layer F.Cu) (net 7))
 (segment (start 132.854 87.872) (end 133.096 87.63) (width 0.25) (layer F.Cu) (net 7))
 (segment (start 134.354 88.646) (end 134.354 96.774) (width 0.25) (layer F.Cu) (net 8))
 (segment (start 134.354 96.774) (end 134.366 96.786) (width 0.25) (layer F.Cu) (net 8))
 (segment (start 136.93902 83.82) (end 136.93902 79.77702) (width 0.25) (layer F.Cu) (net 9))
 (segment (start 136.93902 79.77702) (end 136.918 79.756) (width 0.25) (layer F.Cu) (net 9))
 (segment (start 141.974 79.756) (end 141.974 84.02898) (width 0.25) (layer F.Cu) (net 10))
 (segment (start 141.974 84.02898) (end 142.01902 84.074) (width 0.25) (layer F.Cu) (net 10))
 (segment (start 139.946 88.713) (end 139.946 84.09902) (width 0.25) (layer F.Cu) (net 11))
 (segment (start 139.946 84.09902) (end 139.92098 84.074) (width 0.25) (layer F.Cu) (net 11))
 (segment (start 142.52702 94.742) (end 145.034 94.742) (width 0.25) (layer F.Cu) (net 12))
 (segment (start 146.304 77.724) (end 144.514 77.724) (width 0.25) (layer F.Cu) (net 12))
 (via (at 146.304 77.724) (size 0.6) (drill 0.4) (layers F.Cu B.Cu) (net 12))
 (segment (start 146.304 93.472) (end 146.304 77.724) (width 0.25) (layer B.Cu) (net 12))
 (segment (start 145.034 94.742) (end 146.304 93.472) (width 0.25) (layer B.Cu) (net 12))
 (via (at 145.034 94.742) (size 0.6) (drill 0.4) (layers F.Cu B.Cu) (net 12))
 (segment (start 140.42898 94.742) (end 140.42898 92.66002) (width 0.25) (layer F.Cu) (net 13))
 (segment (start 140.42898 92.66002) (end 140.446 92.643) (width 0.25) (layer F.Cu) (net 13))
 (segment (start 159.766 90.424) (end 160.782 90.424) (width 0.25) (layer B.Cu) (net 14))
 (segment (start 160.782 90.424) (end 161.798 89.408) (width 0.25) (layer B.Cu) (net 14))
 (segment (start 161.798 78.486) (end 161.036 77.724) (width 0.25) (layer F.Cu) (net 14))
 (via (at 161.798 78.486) (size 0.6) (drill 0.4) (layers F.Cu B.Cu) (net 14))
 (segment (start 161.798 89.408) (end 161.798 78.486) (width 0.25) (layer B.Cu) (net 14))
 (segment (start 161.036 77.724) (end 159.766 77.724) (width 0.25) (layer F.Cu) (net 14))
 (segment (start 159.766 90.424) (end 157.734 90.424) (width 0.25) (layer B.Cu) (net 14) (status 10))
 (segment (start 150.876 97.282) (end 149.098 97.282) (width 0.25) (layer F.Cu) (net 14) (status 20))
 (segment (start 152.654 95.504) (end 150.876 97.282) (width 0.25) (layer F.Cu) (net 14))
 (via (at 152.654 95.504) (size 0.6) (drill 0.4) (layers F.Cu B.Cu) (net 14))
 (segment (start 157.734 90.424) (end 152.654 95.504) (width 0.25) (layer B.Cu) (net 14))
 (segment (start 138.446 88.713) (end 138.446 88.662) (width 0.25) (layer F.Cu) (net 20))
 (segment (start 138.446 88.662) (end 136.652 86.868) (width 0.25) (layer F.Cu) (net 20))
 (via (at 136.652 86.868) (size 0.6) (drill 0.4) (layers F.Cu B.Cu) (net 20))
 (segment (start 136.652 86.868) (end 136.652 77.47) (width 0.25) (layer B.Cu) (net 20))
 (segment (start 136.652 77.47) (end 137.16 76.962) (width 0.25) (layer B.Cu) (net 20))
 (segment (start 137.16 76.962) (end 156.464 76.962) (width 0.25) (layer B.Cu) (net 20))
 (segment (start 156.464 76.962) (end 159.766 80.264) (width 0.25) (layer B.Cu) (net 20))
 (segment (start 137.481 91.178) (end 136.406 91.178) (width 0.25) (layer F.Cu) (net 21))
 (segment (start 157.48 85.09) (end 159.766 82.804) (width 0.25) (layer B.Cu) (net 21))
 (segment (start 148.59 85.09) (end 157.48 85.09) (width 0.25) (layer B.Cu) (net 21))
 (segment (start 147.32 86.36) (end 148.59 85.09) (width 0.25) (layer B.Cu) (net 21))
 (via (at 147.32 86.36) (size 0.6) (drill 0.4) (layers F.Cu B.Cu) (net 21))
 (segment (start 145.542 86.36) (end 147.32 86.36) (width 0.25) (layer F.Cu) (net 21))
 (segment (start 144.272 87.63) (end 145.542 86.36) (width 0.25) (layer F.Cu) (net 21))
 (via (at 144.272 87.63) (size 0.6) (drill 0.4) (layers F.Cu B.Cu) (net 21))
 (segment (start 136.652 87.63) (end 144.272 87.63) (width 0.25) (layer B.Cu) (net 21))
 (segment (start 136.398 87.884) (end 136.652 87.63) (width 0.25) (layer B.Cu) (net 21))
 (segment (start 136.398 91.186) (end 136.398 87.884) (width 0.25) (layer B.Cu) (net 21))
 (segment (start 136.144 91.44) (end 136.398 91.186) (width 0.25) (layer B.Cu) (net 21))
 (via (at 136.144 91.44) (size 0.6) (drill 0.4) (layers F.Cu B.Cu) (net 21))
 (segment (start 136.406 91.178) (end 136.144 91.44) (width 0.25) (layer F.Cu) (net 21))
 (segment (start 157.226 86.868) (end 158.242 87.884) (width 0.25) (layer B.Cu) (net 22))
 (via (at 157.226 86.868) (size 0.6) (drill 0.4) (layers F.Cu B.Cu) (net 22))
 (segment (start 154.42 84.062) (end 157.226 86.868) (width 0.25) (layer F.Cu) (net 22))
 (segment (start 154.42 82.55) (end 154.42 84.062) (width 0.25) (layer F.Cu) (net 22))
 (segment (start 158.242 87.884) (end 159.766 87.884) (width 0.25) (layer B.Cu) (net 22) (status 20))
 (segment (start 123.06808 79.89316) (end 123.06808 85.39226) (width 0.25) (layer B.Cu) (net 24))
 (segment (start 114.16792 79.89316) (end 123.06808 79.89316) (width 0.25) (layer B.Cu) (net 24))
 (segment (start 114.16792 85.39226) (end 114.16792 79.89316) (width 0.25) (layer B.Cu) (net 24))
 (segment (start 125.972 91.186) (end 125.972 95.492) (width 0.25) (layer F.Cu) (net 25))
 (segment (start 143.784222 91.240096) (end 141.411 91.178) (width 0.25) (layer F.Cu) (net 25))
 (segment (start 143.792222 91.248096) (end 143.784222 91.240096) (width 0.25) (layer F.Cu) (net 25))
 (via (at 143.792222 91.248096) (size 0.6) (drill 0.4) (layers F.Cu B.Cu) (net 25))
 (segment (start 143.764 96.774) (end 143.792222 91.248096) (width 0.25) (layer B.Cu) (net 25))
 (segment (start 142.748 96.774) (end 143.764 96.774) (width 0.25) (layer B.Cu) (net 25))
 (segment (start 127.254 96.774) (end 142.748 96.774) (width 0.25) (layer B.Cu) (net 25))
 (via (at 127.254 96.774) (size 0.6) (drill 0.4) (layers F.Cu B.Cu) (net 25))
 (segment (start 125.972 95.492) (end 127.254 96.774) (width 0.25) (layer F.Cu) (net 25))
 (segment (start 141.411 91.678) (end 142.994435 91.678) (width 0.25) (layer F.Cu) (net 26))
 (segment (start 130.556 93.98) (end 129.528 93.98) (width 0.25) (layer F.Cu) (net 26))
 (segment (start 132.588 96.012) (end 130.556 93.98) (width 0.25) (layer F.Cu) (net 26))
 (via (at 132.588 96.012) (size 0.6) (drill 0.4) (layers F.Cu B.Cu) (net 26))
 (segment (start 143.002 96.012) (end 132.588 96.012) (width 0.25) (layer B.Cu) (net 26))
 (segment (start 143.002 93.218) (end 143.002 96.012) (width 0.25) (layer B.Cu) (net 26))
 (via (at 143.002 93.218) (size 0.6) (drill 0.4) (layers F.Cu B.Cu) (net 26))
 (segment (start 143.002 91.685565) (end 143.002 93.218) (width 0.25) (layer F.Cu) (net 26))
 (segment (start 142.994435 91.678) (end 143.002 91.685565) (width 0.25) (layer F.Cu) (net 26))
 (segment (start 146.062 79.756) (end 145.288 79.756) (width 0.25) (layer F.Cu) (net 27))
 (segment (start 138.946 87.892) (end 138.946 88.713) (width 0.25) (layer F.Cu) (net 27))
 (segment (start 137.922 86.868) (end 138.946 87.892) (width 0.25) (layer F.Cu) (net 27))
 (via (at 137.922 86.868) (size 0.6) (drill 0.4) (layers F.Cu B.Cu) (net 27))
 (segment (start 137.922 82.296) (end 137.922 86.614) (width 0.25) (layer B.Cu) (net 27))
 (segment (start 137.922 82.296) (end 137.922 82.296) (width 0.25) (layer B.Cu) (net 27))
 (segment (start 142.748 82.296) (end 137.922 82.296) (width 0.25) (layer B.Cu) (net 27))
 (segment (start 143.002 82.042) (end 142.748 82.296) (width 0.25) (layer B.Cu) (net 27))
 (via (at 143.002 82.042) (size 0.6) (drill 0.4) (layers F.Cu B.Cu) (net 27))
 (segment (start 145.288 79.756) (end 143.002 82.042) (width 0.25) (layer F.Cu) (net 27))
 (segment (start 139.446 88.713) (end 139.446 87.122) (width 0.25) (layer F.Cu) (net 28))
 (segment (start 144.272 82.55) (end 152.92 82.55) (width 0.25) (layer F.Cu) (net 28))
 (segment (start 144.018 82.804) (end 144.272 82.55) (width 0.25) (layer F.Cu) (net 28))
 (via (at 144.018 82.804) (size 0.6) (drill 0.4) (layers F.Cu B.Cu) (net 28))
 (segment (start 144.018 84.836) (end 144.018 82.804) (width 0.25) (layer B.Cu) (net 28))
 (segment (start 142.24 86.614) (end 144.018 84.836) (width 0.25) (layer B.Cu) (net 28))
 (segment (start 139.446 86.614) (end 142.24 86.614) (width 0.25) (layer B.Cu) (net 28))
 (segment (start 139.192 86.868) (end 139.446 86.614) (width 0.25) (layer B.Cu) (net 28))
 (via (at 139.192 86.868) (size 0.6) (drill 0.4) (layers F.Cu B.Cu) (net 28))
 (segment (start 139.446 87.122) (end 139.192 86.868) (width 0.25) (layer F.Cu) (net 28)))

